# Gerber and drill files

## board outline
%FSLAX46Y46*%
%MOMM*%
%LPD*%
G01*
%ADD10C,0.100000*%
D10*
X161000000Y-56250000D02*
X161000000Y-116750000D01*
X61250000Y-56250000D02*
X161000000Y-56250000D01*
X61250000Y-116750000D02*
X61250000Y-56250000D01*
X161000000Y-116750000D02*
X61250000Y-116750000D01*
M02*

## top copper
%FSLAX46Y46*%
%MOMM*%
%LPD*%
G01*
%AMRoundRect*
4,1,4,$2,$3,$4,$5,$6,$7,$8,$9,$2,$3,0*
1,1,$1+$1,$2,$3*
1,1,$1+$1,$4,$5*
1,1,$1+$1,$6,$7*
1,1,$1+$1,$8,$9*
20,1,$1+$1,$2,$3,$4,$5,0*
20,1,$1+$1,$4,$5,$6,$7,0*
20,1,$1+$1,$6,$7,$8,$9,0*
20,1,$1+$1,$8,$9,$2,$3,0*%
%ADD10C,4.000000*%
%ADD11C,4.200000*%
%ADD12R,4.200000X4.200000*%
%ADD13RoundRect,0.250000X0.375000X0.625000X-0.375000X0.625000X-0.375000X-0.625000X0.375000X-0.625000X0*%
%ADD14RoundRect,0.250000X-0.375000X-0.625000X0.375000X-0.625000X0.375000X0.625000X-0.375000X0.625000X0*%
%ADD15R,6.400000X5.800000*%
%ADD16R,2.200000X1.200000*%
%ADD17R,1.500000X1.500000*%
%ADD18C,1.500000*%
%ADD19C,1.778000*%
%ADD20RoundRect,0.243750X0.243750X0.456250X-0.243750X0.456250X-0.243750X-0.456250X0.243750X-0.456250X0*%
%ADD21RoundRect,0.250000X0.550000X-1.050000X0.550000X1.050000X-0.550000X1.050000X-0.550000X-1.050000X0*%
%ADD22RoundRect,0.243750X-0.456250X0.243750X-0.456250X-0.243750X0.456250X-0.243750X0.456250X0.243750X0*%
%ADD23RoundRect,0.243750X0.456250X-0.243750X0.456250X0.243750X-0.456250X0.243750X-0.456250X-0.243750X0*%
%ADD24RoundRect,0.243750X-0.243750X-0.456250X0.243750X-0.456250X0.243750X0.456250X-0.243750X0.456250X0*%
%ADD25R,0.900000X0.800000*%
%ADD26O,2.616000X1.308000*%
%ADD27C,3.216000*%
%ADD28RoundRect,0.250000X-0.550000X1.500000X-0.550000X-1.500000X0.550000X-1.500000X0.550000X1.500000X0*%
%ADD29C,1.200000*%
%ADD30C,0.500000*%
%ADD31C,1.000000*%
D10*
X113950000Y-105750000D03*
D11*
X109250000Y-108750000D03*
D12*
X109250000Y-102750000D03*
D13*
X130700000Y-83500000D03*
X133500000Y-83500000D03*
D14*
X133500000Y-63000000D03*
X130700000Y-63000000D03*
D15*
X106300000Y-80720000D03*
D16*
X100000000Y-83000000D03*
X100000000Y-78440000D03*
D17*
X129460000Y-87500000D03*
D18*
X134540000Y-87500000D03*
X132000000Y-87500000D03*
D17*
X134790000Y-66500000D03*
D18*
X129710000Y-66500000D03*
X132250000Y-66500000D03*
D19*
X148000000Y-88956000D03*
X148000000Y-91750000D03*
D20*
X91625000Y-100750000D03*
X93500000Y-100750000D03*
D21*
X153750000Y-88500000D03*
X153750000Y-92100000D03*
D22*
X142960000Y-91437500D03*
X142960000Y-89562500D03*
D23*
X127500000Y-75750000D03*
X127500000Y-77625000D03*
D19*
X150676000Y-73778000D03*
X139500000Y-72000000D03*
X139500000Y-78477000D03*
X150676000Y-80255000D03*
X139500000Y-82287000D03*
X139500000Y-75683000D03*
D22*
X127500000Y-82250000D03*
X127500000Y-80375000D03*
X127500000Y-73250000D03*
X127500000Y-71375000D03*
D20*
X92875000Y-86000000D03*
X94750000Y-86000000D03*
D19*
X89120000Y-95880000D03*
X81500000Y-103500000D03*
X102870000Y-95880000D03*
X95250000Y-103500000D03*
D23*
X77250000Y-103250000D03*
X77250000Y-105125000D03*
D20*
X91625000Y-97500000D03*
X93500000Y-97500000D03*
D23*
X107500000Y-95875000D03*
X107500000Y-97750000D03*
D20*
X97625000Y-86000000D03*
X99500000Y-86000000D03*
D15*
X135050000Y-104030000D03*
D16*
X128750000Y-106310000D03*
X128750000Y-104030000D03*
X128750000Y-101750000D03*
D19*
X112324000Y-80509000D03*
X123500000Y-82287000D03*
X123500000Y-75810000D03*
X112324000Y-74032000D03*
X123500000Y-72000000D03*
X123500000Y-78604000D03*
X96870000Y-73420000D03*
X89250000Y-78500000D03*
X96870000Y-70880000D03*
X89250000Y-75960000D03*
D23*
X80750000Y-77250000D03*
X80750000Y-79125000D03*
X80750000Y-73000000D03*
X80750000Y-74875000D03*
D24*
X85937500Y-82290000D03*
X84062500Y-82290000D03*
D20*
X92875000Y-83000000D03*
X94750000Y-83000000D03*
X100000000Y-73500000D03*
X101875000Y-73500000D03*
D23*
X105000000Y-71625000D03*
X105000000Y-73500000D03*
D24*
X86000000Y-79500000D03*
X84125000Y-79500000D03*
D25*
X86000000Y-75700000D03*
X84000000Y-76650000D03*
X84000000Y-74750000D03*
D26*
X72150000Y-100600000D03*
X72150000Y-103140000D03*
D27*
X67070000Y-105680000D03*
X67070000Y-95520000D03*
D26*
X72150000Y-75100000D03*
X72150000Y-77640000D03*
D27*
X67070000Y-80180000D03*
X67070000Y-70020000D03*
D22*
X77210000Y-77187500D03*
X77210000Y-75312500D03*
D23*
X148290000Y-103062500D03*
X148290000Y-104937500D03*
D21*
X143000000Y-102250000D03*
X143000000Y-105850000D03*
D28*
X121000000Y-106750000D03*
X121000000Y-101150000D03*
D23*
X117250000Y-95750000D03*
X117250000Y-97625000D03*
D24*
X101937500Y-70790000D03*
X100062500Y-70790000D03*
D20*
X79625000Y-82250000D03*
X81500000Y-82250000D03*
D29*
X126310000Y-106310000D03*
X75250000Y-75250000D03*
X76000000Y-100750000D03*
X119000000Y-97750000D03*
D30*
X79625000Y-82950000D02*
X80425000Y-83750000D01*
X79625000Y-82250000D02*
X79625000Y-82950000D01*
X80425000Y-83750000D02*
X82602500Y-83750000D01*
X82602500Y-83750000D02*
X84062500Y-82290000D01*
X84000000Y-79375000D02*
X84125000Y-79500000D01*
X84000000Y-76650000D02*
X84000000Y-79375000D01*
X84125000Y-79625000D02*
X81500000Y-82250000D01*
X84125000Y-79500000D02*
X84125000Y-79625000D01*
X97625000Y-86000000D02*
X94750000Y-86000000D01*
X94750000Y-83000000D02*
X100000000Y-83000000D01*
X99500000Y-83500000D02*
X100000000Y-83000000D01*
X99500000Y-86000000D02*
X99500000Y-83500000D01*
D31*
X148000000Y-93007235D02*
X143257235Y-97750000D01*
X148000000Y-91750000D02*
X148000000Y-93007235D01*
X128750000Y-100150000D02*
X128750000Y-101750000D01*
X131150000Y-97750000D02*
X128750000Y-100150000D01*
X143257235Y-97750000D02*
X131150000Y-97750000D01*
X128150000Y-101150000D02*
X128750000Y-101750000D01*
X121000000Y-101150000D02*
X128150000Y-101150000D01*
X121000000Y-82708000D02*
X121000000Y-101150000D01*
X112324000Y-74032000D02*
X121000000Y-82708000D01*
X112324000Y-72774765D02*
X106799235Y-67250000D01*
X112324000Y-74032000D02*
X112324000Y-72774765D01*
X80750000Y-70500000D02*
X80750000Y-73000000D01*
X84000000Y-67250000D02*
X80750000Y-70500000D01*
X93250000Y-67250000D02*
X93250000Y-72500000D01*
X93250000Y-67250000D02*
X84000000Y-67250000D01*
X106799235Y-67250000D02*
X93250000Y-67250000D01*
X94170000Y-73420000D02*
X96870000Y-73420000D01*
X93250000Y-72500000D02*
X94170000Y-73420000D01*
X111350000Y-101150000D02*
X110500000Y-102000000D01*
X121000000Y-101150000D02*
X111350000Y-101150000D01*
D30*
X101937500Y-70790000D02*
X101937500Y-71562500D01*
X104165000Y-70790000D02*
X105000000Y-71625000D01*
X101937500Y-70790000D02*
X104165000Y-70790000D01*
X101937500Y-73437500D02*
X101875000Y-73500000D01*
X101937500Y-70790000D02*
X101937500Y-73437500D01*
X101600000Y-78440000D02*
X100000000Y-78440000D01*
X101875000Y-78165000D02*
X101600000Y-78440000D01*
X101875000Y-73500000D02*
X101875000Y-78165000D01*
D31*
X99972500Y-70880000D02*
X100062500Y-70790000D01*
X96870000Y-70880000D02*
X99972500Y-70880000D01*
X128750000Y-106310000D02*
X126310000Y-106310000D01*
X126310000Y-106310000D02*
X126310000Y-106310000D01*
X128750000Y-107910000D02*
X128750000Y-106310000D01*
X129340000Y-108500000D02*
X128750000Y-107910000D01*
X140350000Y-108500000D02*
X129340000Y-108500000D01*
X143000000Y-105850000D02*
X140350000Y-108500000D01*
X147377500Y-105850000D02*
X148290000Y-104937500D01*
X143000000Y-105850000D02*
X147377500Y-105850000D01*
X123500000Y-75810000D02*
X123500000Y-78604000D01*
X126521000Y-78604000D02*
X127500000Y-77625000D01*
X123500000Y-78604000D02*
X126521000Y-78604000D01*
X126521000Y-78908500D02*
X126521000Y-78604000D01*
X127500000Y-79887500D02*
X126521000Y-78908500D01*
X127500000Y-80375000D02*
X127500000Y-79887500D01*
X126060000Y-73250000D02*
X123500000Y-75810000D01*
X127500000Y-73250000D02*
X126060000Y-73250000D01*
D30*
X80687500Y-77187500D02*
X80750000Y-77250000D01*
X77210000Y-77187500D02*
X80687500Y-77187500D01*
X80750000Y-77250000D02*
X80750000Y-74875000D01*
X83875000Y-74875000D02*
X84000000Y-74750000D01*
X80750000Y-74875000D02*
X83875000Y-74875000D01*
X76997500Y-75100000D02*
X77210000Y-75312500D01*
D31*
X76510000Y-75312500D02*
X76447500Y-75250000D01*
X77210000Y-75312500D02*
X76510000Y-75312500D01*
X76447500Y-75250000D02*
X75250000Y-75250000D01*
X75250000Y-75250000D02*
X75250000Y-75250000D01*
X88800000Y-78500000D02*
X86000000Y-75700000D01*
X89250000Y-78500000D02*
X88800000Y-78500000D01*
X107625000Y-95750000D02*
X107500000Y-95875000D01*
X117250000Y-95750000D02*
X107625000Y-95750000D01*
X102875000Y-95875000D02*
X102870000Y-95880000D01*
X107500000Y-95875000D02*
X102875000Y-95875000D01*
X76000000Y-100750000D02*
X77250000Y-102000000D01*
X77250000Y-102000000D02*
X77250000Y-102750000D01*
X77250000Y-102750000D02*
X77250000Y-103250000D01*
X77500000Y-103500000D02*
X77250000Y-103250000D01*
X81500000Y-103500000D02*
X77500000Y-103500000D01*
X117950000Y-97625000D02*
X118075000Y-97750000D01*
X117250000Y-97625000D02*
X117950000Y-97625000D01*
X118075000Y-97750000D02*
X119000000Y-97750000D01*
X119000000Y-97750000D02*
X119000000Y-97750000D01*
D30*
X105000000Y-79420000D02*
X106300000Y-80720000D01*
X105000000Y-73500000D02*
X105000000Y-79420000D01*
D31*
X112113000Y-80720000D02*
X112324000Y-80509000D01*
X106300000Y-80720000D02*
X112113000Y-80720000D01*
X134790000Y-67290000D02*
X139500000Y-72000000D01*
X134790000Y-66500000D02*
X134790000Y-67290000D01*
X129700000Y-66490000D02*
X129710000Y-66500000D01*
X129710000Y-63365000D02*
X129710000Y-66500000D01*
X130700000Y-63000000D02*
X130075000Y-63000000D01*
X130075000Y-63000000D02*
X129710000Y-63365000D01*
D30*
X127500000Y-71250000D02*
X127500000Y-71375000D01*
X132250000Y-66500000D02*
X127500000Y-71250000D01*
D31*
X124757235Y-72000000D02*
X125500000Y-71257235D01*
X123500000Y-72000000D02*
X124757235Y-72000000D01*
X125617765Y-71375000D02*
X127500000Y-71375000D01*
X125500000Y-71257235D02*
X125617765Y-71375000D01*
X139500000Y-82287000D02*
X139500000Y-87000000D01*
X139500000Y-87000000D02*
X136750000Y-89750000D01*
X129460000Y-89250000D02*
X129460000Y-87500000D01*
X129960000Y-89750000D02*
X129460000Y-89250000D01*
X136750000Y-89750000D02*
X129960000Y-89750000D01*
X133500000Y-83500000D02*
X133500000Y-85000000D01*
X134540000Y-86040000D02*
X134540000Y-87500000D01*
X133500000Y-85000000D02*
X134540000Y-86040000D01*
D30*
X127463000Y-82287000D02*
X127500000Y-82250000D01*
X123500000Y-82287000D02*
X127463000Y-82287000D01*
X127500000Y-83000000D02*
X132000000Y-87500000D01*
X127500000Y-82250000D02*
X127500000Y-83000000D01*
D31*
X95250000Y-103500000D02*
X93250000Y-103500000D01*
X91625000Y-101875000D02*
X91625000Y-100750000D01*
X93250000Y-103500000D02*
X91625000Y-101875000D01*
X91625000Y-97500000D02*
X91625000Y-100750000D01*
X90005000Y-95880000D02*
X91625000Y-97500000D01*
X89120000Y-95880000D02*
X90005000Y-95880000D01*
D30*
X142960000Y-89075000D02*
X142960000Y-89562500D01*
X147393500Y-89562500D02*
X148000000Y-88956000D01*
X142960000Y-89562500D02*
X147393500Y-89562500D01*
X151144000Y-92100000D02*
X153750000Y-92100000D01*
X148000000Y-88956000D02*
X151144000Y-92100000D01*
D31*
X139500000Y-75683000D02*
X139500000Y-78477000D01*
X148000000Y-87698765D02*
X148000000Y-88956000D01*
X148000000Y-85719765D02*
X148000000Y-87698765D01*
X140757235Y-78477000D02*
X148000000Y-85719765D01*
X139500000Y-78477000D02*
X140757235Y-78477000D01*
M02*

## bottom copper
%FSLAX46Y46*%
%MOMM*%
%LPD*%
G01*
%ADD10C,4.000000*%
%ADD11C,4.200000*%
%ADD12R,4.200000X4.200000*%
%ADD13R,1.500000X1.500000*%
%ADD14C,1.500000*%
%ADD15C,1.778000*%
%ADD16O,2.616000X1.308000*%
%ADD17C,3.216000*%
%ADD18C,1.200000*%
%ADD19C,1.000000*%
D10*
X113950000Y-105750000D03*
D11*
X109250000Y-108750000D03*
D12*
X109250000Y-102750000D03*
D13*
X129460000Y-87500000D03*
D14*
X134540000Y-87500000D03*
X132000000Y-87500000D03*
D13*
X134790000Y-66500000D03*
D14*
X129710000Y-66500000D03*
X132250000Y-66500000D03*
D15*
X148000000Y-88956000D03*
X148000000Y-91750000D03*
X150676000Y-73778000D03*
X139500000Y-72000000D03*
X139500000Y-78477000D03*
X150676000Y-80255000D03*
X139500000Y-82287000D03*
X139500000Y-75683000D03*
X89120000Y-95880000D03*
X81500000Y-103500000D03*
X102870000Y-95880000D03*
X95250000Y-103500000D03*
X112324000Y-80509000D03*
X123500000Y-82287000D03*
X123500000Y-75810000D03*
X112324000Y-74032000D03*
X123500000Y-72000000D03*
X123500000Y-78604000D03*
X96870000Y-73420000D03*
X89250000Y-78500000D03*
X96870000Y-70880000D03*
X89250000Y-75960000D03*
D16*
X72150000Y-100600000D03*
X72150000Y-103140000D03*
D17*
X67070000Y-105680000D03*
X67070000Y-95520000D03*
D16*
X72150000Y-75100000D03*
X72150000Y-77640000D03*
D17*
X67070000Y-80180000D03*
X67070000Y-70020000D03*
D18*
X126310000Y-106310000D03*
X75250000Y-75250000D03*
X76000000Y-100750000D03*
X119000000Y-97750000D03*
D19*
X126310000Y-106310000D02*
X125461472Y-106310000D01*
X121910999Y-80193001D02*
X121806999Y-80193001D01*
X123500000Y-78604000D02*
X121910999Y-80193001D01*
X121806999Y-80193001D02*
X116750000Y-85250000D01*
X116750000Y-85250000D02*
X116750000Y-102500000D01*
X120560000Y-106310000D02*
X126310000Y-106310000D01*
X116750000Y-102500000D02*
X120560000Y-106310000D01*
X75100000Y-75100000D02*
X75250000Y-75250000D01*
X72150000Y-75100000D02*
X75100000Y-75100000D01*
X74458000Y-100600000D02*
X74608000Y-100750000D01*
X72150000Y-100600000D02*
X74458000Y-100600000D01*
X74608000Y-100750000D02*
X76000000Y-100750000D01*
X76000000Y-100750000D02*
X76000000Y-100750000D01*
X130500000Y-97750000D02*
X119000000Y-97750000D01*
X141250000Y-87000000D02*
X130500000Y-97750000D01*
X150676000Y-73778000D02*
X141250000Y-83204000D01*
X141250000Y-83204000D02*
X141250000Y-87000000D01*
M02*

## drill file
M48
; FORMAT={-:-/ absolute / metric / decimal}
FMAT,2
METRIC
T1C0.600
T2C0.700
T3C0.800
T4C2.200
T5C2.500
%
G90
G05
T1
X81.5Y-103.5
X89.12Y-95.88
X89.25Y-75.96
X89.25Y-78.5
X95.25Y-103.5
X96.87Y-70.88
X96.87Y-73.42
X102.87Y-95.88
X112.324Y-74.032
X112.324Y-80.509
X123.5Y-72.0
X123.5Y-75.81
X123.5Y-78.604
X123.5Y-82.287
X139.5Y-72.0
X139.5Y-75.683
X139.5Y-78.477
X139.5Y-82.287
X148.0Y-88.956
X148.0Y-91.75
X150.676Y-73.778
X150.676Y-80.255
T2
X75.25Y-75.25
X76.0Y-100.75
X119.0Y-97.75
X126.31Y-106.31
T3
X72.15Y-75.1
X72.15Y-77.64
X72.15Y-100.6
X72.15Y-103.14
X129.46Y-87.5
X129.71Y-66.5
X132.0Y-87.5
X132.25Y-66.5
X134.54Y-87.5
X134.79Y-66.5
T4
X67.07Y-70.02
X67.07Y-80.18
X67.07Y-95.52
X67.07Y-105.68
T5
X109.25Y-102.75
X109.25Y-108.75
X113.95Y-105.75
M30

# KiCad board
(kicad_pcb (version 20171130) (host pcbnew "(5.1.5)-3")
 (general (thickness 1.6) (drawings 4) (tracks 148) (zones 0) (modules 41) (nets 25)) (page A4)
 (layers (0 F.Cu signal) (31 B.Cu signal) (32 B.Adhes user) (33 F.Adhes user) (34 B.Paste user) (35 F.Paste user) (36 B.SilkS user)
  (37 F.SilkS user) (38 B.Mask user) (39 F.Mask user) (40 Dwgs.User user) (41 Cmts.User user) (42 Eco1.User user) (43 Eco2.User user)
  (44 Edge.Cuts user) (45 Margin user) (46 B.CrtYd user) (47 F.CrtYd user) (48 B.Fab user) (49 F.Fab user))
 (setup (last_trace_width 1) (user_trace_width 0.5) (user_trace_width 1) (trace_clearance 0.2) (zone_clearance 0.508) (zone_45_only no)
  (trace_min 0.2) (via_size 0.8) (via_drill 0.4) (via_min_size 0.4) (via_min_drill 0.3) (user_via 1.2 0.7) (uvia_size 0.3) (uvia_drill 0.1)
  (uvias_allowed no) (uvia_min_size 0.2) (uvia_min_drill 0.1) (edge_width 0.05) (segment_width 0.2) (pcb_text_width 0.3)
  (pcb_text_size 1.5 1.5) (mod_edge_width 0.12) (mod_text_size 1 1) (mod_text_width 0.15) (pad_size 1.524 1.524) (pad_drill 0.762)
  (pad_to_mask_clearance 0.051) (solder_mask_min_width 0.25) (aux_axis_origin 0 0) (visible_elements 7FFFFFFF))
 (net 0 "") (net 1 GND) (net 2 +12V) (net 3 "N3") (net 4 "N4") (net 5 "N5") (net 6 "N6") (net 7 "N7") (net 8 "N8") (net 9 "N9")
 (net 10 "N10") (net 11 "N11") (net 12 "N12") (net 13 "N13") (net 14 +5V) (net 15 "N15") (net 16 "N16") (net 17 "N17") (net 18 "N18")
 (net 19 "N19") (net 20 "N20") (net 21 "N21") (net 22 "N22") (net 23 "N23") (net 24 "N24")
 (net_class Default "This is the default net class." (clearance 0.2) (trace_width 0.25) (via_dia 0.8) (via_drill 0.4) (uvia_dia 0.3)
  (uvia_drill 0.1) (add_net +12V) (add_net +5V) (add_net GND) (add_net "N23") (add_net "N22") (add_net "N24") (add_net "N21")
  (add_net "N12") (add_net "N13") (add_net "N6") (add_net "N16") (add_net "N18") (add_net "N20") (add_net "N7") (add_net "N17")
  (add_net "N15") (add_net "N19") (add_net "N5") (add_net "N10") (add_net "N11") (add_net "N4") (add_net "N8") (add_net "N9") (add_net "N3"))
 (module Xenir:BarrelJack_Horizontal (layer F.Cu) (at 109.25 102.75)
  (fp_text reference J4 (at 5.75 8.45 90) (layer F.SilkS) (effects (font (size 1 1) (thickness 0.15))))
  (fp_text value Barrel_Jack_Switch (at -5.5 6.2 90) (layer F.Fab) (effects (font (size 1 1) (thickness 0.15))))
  (pad 3 thru_hole circle (at 4.7 3) (size 4 4) (drill 2.5) (layers *.Cu *.Mask))
  (pad 2 thru_hole circle (at 0 6) (size 4.2 4.2) (drill 2.5) (layers *.Cu *.Mask) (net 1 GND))
  (pad 1 thru_hole rect (at 0 0) (size 4.2 4.2) (drill 2.5) (layers *.Cu *.Mask) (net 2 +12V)))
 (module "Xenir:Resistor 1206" (layer F.Cu) (at 131.973 85.877 180)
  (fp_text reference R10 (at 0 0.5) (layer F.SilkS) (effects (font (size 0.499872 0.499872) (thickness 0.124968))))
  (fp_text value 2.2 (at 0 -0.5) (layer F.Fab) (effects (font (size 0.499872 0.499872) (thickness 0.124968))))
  (pad 2 smd roundrect (at 1.273 2.377 180) (size 1.25 1.75) (layers F.Cu F.Paste F.Mask) (roundrect_rratio 0.2) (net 1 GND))
  (pad 1 smd roundrect (at -1.527 2.377 180) (size 1.25 1.75) (layers F.Cu F.Paste F.Mask) (roundrect_rratio 0.2) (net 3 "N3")))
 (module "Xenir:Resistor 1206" (layer F.Cu) (at 132.227 60.623)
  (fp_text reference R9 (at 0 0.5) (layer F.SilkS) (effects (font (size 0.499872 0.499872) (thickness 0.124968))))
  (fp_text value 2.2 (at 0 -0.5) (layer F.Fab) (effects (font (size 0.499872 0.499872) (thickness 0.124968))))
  (pad 2 smd roundrect (at 1.273 2.377) (size 1.25 1.75) (layers F.Cu F.Paste F.Mask) (roundrect_rratio 0.2) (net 1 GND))
  (pad 1 smd roundrect (at -1.527 2.377) (size 1.25 1.75) (layers F.Cu F.Paste F.Mask) (roundrect_rratio 0.2) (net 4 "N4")))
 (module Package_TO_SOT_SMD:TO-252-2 (layer F.Cu) (at 104.2 80.72)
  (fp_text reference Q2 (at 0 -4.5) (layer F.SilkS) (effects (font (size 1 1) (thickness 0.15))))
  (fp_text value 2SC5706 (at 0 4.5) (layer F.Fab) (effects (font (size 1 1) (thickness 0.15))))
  (pad "" smd rect (at 0.425 1.525) (size 3.05 2.75) (layers F.Paste))
  (pad "" smd rect (at 3.775 -1.525) (size 3.05 2.75) (layers F.Paste))
  (pad "" smd rect (at 0.425 -1.525) (size 3.05 2.75) (layers F.Paste))
  (pad "" smd rect (at 3.775 1.525) (size 3.05 2.75) (layers F.Paste))
  (pad 2 smd rect (at 2.1 0) (size 6.4 5.8) (layers F.Cu F.Mask) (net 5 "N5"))
  (pad 3 smd rect (at -4.2 2.28) (size 2.2 1.2) (layers F.Cu F.Paste F.Mask) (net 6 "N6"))
  (pad 1 smd rect (at -4.2 -2.28) (size 2.2 1.2) (layers F.Cu F.Paste F.Mask) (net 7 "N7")))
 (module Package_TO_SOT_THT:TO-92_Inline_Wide (layer F.Cu) (at 129.46 87.5)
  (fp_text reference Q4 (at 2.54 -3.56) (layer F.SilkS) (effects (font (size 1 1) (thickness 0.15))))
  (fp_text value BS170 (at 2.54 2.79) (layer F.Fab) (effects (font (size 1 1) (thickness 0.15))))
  (pad 1 thru_hole rect (at 0 0 90) (size 1.5 1.5) (drill 0.8) (layers *.Cu *.Mask) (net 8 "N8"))
  (pad 3 thru_hole circle (at 5.08 0 90) (size 1.5 1.5) (drill 0.8) (layers *.Cu *.Mask) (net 3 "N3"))
  (pad 2 thru_hole circle (at 2.54 0 90) (size 1.5 1.5) (drill 0.8) (layers *.Cu *.Mask) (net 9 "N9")))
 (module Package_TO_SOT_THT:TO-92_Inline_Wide (layer F.Cu) (at 134.79 66.5 180)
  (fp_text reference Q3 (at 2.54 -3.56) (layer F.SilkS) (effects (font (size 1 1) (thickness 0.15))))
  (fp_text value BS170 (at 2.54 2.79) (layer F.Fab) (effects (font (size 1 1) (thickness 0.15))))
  (pad 1 thru_hole rect (at 0 0 270) (size 1.5 1.5) (drill 0.8) (layers *.Cu *.Mask) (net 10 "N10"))
  (pad 3 thru_hole circle (at 5.08 0 270) (size 1.5 1.5) (drill 0.8) (layers *.Cu *.Mask) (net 4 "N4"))
  (pad 2 thru_hole circle (at 2.54 0 270) (size 1.5 1.5) (drill 0.8) (layers *.Cu *.Mask) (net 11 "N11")))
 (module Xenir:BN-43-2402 (layer F.Cu) (at 148 95.687 180)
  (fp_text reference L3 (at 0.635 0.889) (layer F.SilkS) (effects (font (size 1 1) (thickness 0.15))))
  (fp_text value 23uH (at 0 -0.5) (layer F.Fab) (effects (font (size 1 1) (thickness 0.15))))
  (pad 2 thru_hole circle (at 0 6.731 180) (size 1.778 1.778) (drill 0.6) (layers *.Cu *.Mask) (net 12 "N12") (solder_mask_margin 0.1016))
  (pad 1 thru_hole circle (at 0 3.937 180) (size 1.778 1.778) (drill 0.6) (layers *.Cu *.Mask) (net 2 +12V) (solder_mask_margin 0.1016)))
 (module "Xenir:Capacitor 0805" (layer F.Cu) (at 92.5625 103.29 180)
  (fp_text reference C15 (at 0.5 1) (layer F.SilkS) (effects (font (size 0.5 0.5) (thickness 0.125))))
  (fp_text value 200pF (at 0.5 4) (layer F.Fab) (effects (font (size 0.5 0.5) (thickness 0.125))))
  (pad 2 smd roundrect (at 0.9375 2.54 180) (size 0.975 1.4) (layers F.Cu F.Paste F.Mask) (roundrect_rratio 0.25) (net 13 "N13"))
  (pad 1 smd roundrect (at -0.9375 2.54 180) (size 0.975 1.4) (layers F.Cu F.Paste F.Mask) (roundrect_rratio 0.25) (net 1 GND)))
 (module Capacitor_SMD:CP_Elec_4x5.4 (layer F.Cu) (at 153.75 90.3 90)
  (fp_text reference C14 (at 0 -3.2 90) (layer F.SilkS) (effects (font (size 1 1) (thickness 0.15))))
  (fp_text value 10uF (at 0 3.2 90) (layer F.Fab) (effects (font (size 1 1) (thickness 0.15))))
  (pad 2 smd roundrect (at 1.8 0 90) (size 2.6 1.6) (layers F.Cu F.Paste F.Mask) (roundrect_rratio 0.15625) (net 1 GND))
  (pad 1 smd roundrect (at -1.8 0 90) (size 2.6 1.6) (layers F.Cu F.Paste F.Mask) (roundrect_rratio 0.15625) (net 12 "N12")))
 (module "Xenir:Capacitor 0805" (layer F.Cu) (at 145.5 90.5 270)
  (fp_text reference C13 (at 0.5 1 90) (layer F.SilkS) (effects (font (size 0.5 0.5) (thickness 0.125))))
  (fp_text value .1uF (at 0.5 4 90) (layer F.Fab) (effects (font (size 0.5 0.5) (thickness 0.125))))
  (pad 2 smd roundrect (at 0.9375 2.54 270) (size 0.975 1.4) (layers F.Cu F.Paste F.Mask) (roundrect_rratio 0.25) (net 1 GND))
  (pad 1 smd roundrect (at -0.9375 2.54 270) (size 0.975 1.4) (layers F.Cu F.Paste F.Mask) (roundrect_rratio 0.25) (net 12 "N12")))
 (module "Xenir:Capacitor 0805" (layer F.Cu) (at 124.96 76.6875 90)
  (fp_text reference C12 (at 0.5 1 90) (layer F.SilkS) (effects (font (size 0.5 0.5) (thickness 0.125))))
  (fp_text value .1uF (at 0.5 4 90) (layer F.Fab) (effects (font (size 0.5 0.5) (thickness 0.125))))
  (pad 2 smd roundrect (at 0.9375 2.54 90) (size 0.975 1.4) (layers F.Cu F.Paste F.Mask) (roundrect_rratio 0.25) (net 1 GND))
  (pad 1 smd roundrect (at -0.9375 2.54 90) (size 0.975 1.4) (layers F.Cu F.Paste F.Mask) (roundrect_rratio 0.25) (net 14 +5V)))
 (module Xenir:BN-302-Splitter (layer F.Cu) (at 145.088 85.843 180)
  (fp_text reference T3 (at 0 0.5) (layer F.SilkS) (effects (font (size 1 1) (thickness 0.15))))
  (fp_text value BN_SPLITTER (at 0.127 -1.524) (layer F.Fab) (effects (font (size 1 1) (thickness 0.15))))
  (pad C1B thru_hole circle (at -5.588 12.065 180) (size 1.778 1.778) (drill 0.6) (layers *.Cu *.Mask) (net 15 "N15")
   (solder_mask_margin 0.1016))
  (pad C3B thru_hole circle (at 5.588 13.843 180) (size 1.778 1.778) (drill 0.6) (layers *.Cu *.Mask) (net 10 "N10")
   (solder_mask_margin 0.1016))
  (pad C2B thru_hole circle (at 5.588 7.366 180) (size 1.778 1.778) (drill 0.6) (layers *.Cu *.Mask) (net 12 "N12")
   (solder_mask_margin 0.1016))
  (pad C1A thru_hole circle (at -5.588 5.588 180) (size 1.778 1.778) (drill 0.6) (layers *.Cu *.Mask) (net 1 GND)
   (solder_mask_margin 0.1016))
  (pad C2A thru_hole circle (at 5.588 3.556 180) (size 1.778 1.778) (drill 0.6) (layers *.Cu *.Mask) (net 8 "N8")
   (solder_mask_margin 0.1016))
  (pad C3A thru_hole circle (at 5.588 10.16 180) (size 1.778 1.778) (drill 0.6) (layers *.Cu *.Mask) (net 12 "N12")
   (solder_mask_margin 0.1016)))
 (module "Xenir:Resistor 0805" (layer F.Cu) (at 130.04 81.3125 270)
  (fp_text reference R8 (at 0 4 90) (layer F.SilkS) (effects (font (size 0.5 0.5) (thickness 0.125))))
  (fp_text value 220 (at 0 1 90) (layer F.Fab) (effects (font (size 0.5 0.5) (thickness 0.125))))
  (pad 2 smd roundrect (at 0.9375 2.54 270) (size 0.975 1.4) (layers F.Cu F.Paste F.Mask) (roundrect_rratio 0.25) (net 9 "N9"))
  (pad 1 smd roundrect (at -0.9375 2.54 270) (size 0.975 1.4) (layers F.Cu F.Paste F.Mask) (roundrect_rratio 0.25) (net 14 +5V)))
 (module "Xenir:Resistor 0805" (layer F.Cu) (at 130.04 72.3125 270)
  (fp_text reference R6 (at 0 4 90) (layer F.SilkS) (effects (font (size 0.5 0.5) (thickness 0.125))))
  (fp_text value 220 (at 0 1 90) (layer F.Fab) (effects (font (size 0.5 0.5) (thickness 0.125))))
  (pad 2 smd roundrect (at 0.9375 2.54 270) (size 0.975 1.4) (layers F.Cu F.Paste F.Mask) (roundrect_rratio 0.25) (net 14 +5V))
  (pad 1 smd roundrect (at -0.9375 2.54 270) (size 0.975 1.4) (layers F.Cu F.Paste F.Mask) (roundrect_rratio 0.25) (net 11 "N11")))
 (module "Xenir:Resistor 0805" (layer F.Cu) (at 93.8125 88.54 180)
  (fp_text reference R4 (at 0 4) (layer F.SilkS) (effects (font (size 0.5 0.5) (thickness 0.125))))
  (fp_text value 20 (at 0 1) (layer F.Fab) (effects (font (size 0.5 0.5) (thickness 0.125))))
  (pad 2 smd roundrect (at 0.9375 2.54 180) (size 0.975 1.4) (layers F.Cu F.Paste F.Mask) (roundrect_rratio 0.25) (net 1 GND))
  (pad 1 smd roundrect (at -0.9375 2.54 180) (size 0.975 1.4) (layers F.Cu F.Paste F.Mask) (roundrect_rratio 0.25) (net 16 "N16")))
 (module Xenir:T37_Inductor (layer F.Cu) (at 85.31 106.69 180)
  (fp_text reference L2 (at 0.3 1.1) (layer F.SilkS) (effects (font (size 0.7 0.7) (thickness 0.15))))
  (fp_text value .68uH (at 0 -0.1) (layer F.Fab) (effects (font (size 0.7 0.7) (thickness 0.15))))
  (pad 1 thru_hole circle (at -3.81 10.81 180) (size 1.778 1.778) (drill 0.6) (layers *.Cu *.Mask) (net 13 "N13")
   (solder_mask_margin 0.1016))
  (pad 2 thru_hole circle (at 3.81 3.19 180) (size 1.778 1.778) (drill 0.6) (layers *.Cu *.Mask) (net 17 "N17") (solder_mask_margin 0.1016)))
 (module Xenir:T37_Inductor (layer F.Cu) (at 99.06 106.69 180)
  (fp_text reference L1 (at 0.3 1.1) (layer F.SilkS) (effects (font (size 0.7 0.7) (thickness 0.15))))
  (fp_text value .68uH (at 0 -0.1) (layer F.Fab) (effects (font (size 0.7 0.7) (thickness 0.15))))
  (pad 1 thru_hole circle (at -3.81 10.81 180) (size 1.778 1.778) (drill 0.6) (layers *.Cu *.Mask) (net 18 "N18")
   (solder_mask_margin 0.1016))
  (pad 2 thru_hole circle (at 3.81 3.19 180) (size 1.778 1.778) (drill 0.6) (layers *.Cu *.Mask) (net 13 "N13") (solder_mask_margin 0.1016)))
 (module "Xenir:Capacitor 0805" (layer F.Cu) (at 74.71 104.1875 90)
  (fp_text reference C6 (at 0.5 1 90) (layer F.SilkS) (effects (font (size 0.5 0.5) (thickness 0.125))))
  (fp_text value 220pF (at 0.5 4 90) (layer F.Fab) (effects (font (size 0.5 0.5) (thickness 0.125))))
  (pad 2 smd roundrect (at 0.9375 2.54 90) (size 0.975 1.4) (layers F.Cu F.Paste F.Mask) (roundrect_rratio 0.25) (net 17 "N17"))
  (pad 1 smd roundrect (at -0.9375 2.54 90) (size 0.975 1.4) (layers F.Cu F.Paste F.Mask) (roundrect_rratio 0.25) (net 1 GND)))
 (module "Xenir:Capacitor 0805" (layer F.Cu) (at 92.5625 100.04 180)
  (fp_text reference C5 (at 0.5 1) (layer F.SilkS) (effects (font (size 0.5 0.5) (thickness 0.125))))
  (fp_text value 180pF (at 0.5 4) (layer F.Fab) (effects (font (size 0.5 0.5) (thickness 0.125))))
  (pad 2 smd roundrect (at 0.9375 2.54 180) (size 0.975 1.4) (layers F.Cu F.Paste F.Mask) (roundrect_rratio 0.25) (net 13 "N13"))
  (pad 1 smd roundrect (at -0.9375 2.54 180) (size 0.975 1.4) (layers F.Cu F.Paste F.Mask) (roundrect_rratio 0.25) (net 1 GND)))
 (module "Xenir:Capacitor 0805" (layer F.Cu) (at 104.96 96.8125 90)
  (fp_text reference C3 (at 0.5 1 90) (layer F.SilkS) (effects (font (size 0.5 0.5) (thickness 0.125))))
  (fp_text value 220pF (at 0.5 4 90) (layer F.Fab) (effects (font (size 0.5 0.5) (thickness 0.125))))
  (pad 2 smd roundrect (at 0.9375 2.54 90) (size 0.975 1.4) (layers F.Cu F.Paste F.Mask) (roundrect_rratio 0.25) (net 18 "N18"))
  (pad 1 smd roundrect (at -0.9375 2.54 90) (size 0.975 1.4) (layers F.Cu F.Paste F.Mask) (roundrect_rratio 0.25) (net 1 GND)))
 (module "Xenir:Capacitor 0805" (layer F.Cu) (at 98.5625 88.54 180)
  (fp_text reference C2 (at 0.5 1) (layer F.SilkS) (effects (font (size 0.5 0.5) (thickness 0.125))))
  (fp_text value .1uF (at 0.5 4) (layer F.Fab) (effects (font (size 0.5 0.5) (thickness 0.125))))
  (pad 2 smd roundrect (at 0.9375 2.54 180) (size 0.975 1.4) (layers F.Cu F.Paste F.Mask) (roundrect_rratio 0.25) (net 16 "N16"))
  (pad 1 smd roundrect (at -0.9375 2.54 180) (size 0.975 1.4) (layers F.Cu F.Paste F.Mask) (roundrect_rratio 0.25) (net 6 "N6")))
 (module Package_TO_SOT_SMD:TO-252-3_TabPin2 (layer F.Cu) (at 132.95 104.03)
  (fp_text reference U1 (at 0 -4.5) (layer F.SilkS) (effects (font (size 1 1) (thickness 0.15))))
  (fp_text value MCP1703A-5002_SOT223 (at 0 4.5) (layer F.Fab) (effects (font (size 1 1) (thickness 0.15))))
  (pad "" smd rect (at 0.425 1.525) (size 3.05 2.75) (layers F.Paste))
  (pad "" smd rect (at 3.775 -1.525) (size 3.05 2.75) (layers F.Paste))
  (pad "" smd rect (at 0.425 -1.525) (size 3.05 2.75) (layers F.Paste))
  (pad "" smd rect (at 3.775 1.525) (size 3.05 2.75) (layers F.Paste))
  (pad 2 smd rect (at 2.1 0) (size 6.4 5.8) (layers F.Cu F.Mask) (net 1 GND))
  (pad 3 smd rect (at -4.2 2.28) (size 2.2 1.2) (layers F.Cu F.Paste F.Mask) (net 14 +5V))
  (pad 2 smd rect (at -4.2 0) (size 2.2 1.2) (layers F.Cu F.Paste F.Mask) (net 1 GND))
  (pad 1 smd rect (at -4.2 -2.28) (size 2.2 1.2) (layers F.Cu F.Paste F.Mask) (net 2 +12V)))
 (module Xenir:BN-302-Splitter (layer F.Cu) (at 117.912 68.444)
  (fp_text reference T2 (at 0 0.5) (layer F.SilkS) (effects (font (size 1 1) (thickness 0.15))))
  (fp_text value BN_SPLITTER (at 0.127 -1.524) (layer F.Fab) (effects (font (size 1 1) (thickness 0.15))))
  (pad C1B thru_hole circle (at -5.588 12.065) (size 1.778 1.778) (drill 0.6) (layers *.Cu *.Mask) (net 5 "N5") (solder_mask_margin 0.1016))
  (pad C3B thru_hole circle (at 5.588 13.843) (size 1.778 1.778) (drill 0.6) (layers *.Cu *.Mask) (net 9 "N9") (solder_mask_margin 0.1016))
  (pad C2B thru_hole circle (at 5.588 7.366) (size 1.778 1.778) (drill 0.6) (layers *.Cu *.Mask) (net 14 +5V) (solder_mask_margin 0.1016))
  (pad C1A thru_hole circle (at -5.588 5.588) (size 1.778 1.778) (drill 0.6) (layers *.Cu *.Mask) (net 2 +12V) (solder_mask_margin 0.1016))
  (pad C2A thru_hole circle (at 5.588 3.556) (size 1.778 1.778) (drill 0.6) (layers *.Cu *.Mask) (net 11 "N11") (solder_mask_margin 0.1016))
  (pad C3A thru_hole circle (at 5.588 10.16) (size 1.778 1.778) (drill 0.6) (layers *.Cu *.Mask) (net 14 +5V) (solder_mask_margin 0.1016)))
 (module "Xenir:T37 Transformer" (layer F.Cu) (at 93.06 67.69)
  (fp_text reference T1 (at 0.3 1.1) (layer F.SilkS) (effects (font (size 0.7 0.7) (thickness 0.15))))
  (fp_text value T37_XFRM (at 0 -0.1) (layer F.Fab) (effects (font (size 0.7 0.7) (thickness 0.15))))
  (pad C1B thru_hole circle (at 3.81 5.73) (size 1.778 1.778) (drill 0.6) (layers *.Cu *.Mask) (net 2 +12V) (solder_mask_margin 0.1016))
  (pad C1A thru_hole circle (at -3.81 10.81) (size 1.778 1.778) (drill 0.6) (layers *.Cu *.Mask) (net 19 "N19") (solder_mask_margin 0.1016))
  (pad C2B thru_hole circle (at 3.81 3.19) (size 1.778 1.778) (drill 0.6) (layers *.Cu *.Mask) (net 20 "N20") (solder_mask_margin 0.1016))
  (pad C2A thru_hole circle (at -3.81 8.27) (size 1.778 1.778) (drill 0.6) (layers *.Cu *.Mask) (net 1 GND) (solder_mask_margin 0.1016)))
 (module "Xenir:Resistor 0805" (layer F.Cu) (at 78.21 78.1875 90)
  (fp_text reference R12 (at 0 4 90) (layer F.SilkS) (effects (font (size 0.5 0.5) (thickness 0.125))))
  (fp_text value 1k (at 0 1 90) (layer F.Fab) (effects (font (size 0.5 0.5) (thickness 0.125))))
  (pad 2 smd roundrect (at 0.9375 2.54 90) (size 0.975 1.4) (layers F.Cu F.Paste F.Mask) (roundrect_rratio 0.25) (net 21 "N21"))
  (pad 1 smd roundrect (at -0.9375 2.54 90) (size 0.975 1.4) (layers F.Cu F.Paste F.Mask) (roundrect_rratio 0.25) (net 1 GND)))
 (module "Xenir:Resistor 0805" (layer F.Cu) (at 78.21 73.9375 90)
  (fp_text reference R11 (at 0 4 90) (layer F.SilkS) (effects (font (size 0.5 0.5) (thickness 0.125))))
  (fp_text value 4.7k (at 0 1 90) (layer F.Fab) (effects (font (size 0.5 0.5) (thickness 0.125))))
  (pad 2 smd roundrect (at 0.9375 2.54 90) (size 0.975 1.4) (layers F.Cu F.Paste F.Mask) (roundrect_rratio 0.25) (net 2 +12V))
  (pad 1 smd roundrect (at -0.9375 2.54 90) (size 0.975 1.4) (layers F.Cu F.Paste F.Mask) (roundrect_rratio 0.25) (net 21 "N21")))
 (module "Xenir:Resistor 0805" (layer F.Cu) (at 85 79.75)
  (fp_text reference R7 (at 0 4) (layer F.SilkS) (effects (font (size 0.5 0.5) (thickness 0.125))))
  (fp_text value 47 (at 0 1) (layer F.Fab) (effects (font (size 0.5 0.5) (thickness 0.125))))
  (pad 2 smd roundrect (at 0.9375 2.54) (size 0.975 1.4) (layers F.Cu F.Paste F.Mask) (roundrect_rratio 0.25) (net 1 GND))
  (pad 1 smd roundrect (at -0.9375 2.54) (size 0.975 1.4) (layers F.Cu F.Paste F.Mask) (roundrect_rratio 0.25) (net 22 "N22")))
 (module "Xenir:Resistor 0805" (layer F.Cu) (at 93.8125 85.54 180)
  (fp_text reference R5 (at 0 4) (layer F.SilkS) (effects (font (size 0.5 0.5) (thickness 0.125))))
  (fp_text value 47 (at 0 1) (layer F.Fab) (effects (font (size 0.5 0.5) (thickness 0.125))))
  (pad 2 smd roundrect (at 0.9375 2.54 180) (size 0.975 1.4) (layers F.Cu F.Paste F.Mask) (roundrect_rratio 0.25) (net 1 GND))
  (pad 1 smd roundrect (at -0.9375 2.54 180) (size 0.975 1.4) (layers F.Cu F.Paste F.Mask) (roundrect_rratio 0.25) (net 6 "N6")))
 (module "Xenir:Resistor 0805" (layer F.Cu) (at 100.9375 76.04 180)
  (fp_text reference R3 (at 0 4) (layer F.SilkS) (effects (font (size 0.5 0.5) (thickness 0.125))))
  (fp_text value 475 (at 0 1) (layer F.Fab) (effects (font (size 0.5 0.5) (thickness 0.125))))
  (pad 2 smd roundrect (at 0.9375 2.54 180) (size 0.975 1.4) (layers F.Cu F.Paste F.Mask) (roundrect_rratio 0.25) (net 1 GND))
  (pad 1 smd roundrect (at -0.9375 2.54 180) (size 0.975 1.4) (layers F.Cu F.Paste F.Mask) (roundrect_rratio 0.25) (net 7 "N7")))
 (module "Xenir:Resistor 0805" (layer F.Cu) (at 102.46 72.5625 90)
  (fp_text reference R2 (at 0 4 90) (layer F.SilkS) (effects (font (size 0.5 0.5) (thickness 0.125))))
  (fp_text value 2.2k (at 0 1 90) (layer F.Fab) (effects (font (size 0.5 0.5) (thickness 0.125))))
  (pad 2 smd roundrect (at 0.9375 2.54 90) (size 0.975 1.4) (layers F.Cu F.Paste F.Mask) (roundrect_rratio 0.25) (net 7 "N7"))
  (pad 1 smd roundrect (at -0.9375 2.54 90) (size 0.975 1.4) (layers F.Cu F.Paste F.Mask) (roundrect_rratio 0.25) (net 5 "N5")))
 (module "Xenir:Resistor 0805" (layer F.Cu) (at 85.0625 76.96)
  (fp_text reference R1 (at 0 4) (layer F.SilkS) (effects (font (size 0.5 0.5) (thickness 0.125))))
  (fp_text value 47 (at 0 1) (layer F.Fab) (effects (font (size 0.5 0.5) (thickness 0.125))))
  (pad 2 smd roundrect (at 0.9375 2.54) (size 0.975 1.4) (layers F.Cu F.Paste F.Mask) (roundrect_rratio 0.25) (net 1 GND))
  (pad 1 smd roundrect (at -0.9375 2.54) (size 0.975 1.4) (layers F.Cu F.Paste F.Mask) (roundrect_rratio 0.25) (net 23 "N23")))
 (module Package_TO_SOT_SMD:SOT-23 (layer F.Cu) (at 85 75.7)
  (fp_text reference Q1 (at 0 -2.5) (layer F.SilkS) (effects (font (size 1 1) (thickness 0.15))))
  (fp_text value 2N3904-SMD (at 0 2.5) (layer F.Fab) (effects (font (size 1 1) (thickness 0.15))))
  (pad 3 smd rect (at 1 0) (size 0.9 0.8) (layers F.Cu F.Paste F.Mask) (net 19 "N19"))
  (pad 2 smd rect (at -1 0.95) (size 0.9 0.8) (layers F.Cu F.Paste F.Mask) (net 23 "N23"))
  (pad 1 smd rect (at -1 -0.95) (size 0.9 0.8) (layers F.Cu F.Paste F.Mask) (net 21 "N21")))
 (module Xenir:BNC (layer F.Cu) (at 68.25 100.5 90)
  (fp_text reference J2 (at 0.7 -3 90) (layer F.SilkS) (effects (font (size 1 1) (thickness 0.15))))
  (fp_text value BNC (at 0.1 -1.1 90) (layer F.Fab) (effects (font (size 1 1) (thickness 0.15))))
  (pad S thru_hole oval (at -0.1 3.9 180) (size 2.616 1.308) (drill 0.8) (layers *.Cu *.Mask) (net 17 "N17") (solder_mask_margin 0.1016))
  (pad GND thru_hole oval (at -2.64 3.9 180) (size 2.616 1.308) (drill 0.8) (layers *.Cu *.Mask) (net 1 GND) (solder_mask_margin 0.1016))
  (pad 3 thru_hole circle (at -5.18 -1.18 90) (size 3.216 3.216) (drill 2.2) (layers *.Cu *.Mask) (solder_mask_margin 0.1016))
  (pad 4 thru_hole circle (at 4.98 -1.18 90) (size 3.216 3.216) (drill 2.2) (layers *.Cu *.Mask) (solder_mask_margin 0.1016)))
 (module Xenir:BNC (layer F.Cu) (at 68.25 75 90)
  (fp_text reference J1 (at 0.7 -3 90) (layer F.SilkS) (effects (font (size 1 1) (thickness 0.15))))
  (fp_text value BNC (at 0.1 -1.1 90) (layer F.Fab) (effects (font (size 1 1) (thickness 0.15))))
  (pad S thru_hole oval (at -0.1 3.9 180) (size 2.616 1.308) (drill 0.8) (layers *.Cu *.Mask) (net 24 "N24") (solder_mask_margin 0.1016))
  (pad GND thru_hole oval (at -2.64 3.9 180) (size 2.616 1.308) (drill 0.8) (layers *.Cu *.Mask) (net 1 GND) (solder_mask_margin 0.1016))
  (pad 3 thru_hole circle (at -5.18 -1.18 90) (size 3.216 3.216) (drill 2.2) (layers *.Cu *.Mask) (solder_mask_margin 0.1016))
  (pad 4 thru_hole circle (at 4.98 -1.18 90) (size 3.216 3.216) (drill 2.2) (layers *.Cu *.Mask) (solder_mask_margin 0.1016)))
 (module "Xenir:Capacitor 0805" (layer F.Cu) (at 79.75 76.25 270)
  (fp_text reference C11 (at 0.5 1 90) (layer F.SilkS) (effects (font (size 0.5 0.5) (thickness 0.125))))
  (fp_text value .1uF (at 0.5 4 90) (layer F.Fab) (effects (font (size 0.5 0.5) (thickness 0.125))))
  (pad 2 smd roundrect (at 0.9375 2.54 270) (size 0.975 1.4) (layers F.Cu F.Paste F.Mask) (roundrect_rratio 0.25) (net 21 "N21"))
  (pad 1 smd roundrect (at -0.9375 2.54 270) (size 0.975 1.4) (layers F.Cu F.Paste F.Mask) (roundrect_rratio 0.25) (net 24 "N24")))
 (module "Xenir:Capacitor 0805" (layer F.Cu) (at 145.75 104 90)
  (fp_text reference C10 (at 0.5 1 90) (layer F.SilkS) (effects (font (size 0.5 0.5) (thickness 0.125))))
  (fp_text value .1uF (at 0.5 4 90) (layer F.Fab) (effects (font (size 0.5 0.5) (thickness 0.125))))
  (pad 2 smd roundrect (at 0.9375 2.54 90) (size 0.975 1.4) (layers F.Cu F.Paste F.Mask) (roundrect_rratio 0.25) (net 1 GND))
  (pad 1 smd roundrect (at -0.9375 2.54 90) (size 0.975 1.4) (layers F.Cu F.Paste F.Mask) (roundrect_rratio 0.25) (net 14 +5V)))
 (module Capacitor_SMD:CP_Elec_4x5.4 (layer F.Cu) (at 143 104.05 90)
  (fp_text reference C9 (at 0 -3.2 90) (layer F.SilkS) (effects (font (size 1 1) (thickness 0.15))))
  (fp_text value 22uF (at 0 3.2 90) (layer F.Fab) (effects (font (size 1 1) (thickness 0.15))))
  (pad 2 smd roundrect (at 1.8 0 90) (size 2.6 1.6) (layers F.Cu F.Paste F.Mask) (roundrect_rratio 0.15625) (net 1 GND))
  (pad 1 smd roundrect (at -1.8 0 90) (size 2.6 1.6) (layers F.Cu F.Paste F.Mask) (roundrect_rratio 0.15625) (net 14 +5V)))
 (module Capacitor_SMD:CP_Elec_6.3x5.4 (layer F.Cu) (at 121 103.95 270)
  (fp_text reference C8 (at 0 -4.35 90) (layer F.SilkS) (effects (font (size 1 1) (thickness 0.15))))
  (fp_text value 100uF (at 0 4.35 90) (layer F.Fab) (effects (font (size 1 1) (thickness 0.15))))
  (pad 2 smd roundrect (at 2.8 0 270) (size 3.5 1.6) (layers F.Cu F.Paste F.Mask) (roundrect_rratio 0.15625) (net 1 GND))
  (pad 1 smd roundrect (at -2.8 0 270) (size 3.5 1.6) (layers F.Cu F.Paste F.Mask) (roundrect_rratio 0.15625) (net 2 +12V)))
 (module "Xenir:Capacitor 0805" (layer F.Cu) (at 114.71 96.6875 90)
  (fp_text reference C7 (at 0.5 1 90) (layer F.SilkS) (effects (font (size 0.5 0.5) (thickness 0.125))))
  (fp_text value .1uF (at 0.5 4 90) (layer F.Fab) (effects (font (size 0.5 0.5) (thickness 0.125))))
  (pad 2 smd roundrect (at 0.9375 2.54 90) (size 0.975 1.4) (layers F.Cu F.Paste F.Mask) (roundrect_rratio 0.25) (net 18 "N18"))
  (pad 1 smd roundrect (at -0.9375 2.54 90) (size 0.975 1.4) (layers F.Cu F.Paste F.Mask) (roundrect_rratio 0.25) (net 15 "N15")))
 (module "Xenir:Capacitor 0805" (layer F.Cu) (at 101 68.25)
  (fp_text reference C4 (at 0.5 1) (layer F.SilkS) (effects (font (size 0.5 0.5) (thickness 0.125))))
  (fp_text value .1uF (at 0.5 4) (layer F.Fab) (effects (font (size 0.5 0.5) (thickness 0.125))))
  (pad 2 smd roundrect (at 0.9375 2.54) (size 0.975 1.4) (layers F.Cu F.Paste F.Mask) (roundrect_rratio 0.25) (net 7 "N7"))
  (pad 1 smd roundrect (at -0.9375 2.54) (size 0.975 1.4) (layers F.Cu F.Paste F.Mask) (roundrect_rratio 0.25) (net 20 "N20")))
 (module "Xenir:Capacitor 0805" (layer F.Cu) (at 80.5625 84.79 180)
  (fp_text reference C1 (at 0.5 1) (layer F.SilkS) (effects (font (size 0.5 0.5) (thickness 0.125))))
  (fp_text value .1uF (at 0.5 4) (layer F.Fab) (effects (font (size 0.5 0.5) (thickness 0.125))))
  (pad 2 smd roundrect (at 0.9375 2.54 180) (size 0.975 1.4) (layers F.Cu F.Paste F.Mask) (roundrect_rratio 0.25) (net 22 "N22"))
  (pad 1 smd roundrect (at -0.9375 2.54 180) (size 0.975 1.4) (layers F.Cu F.Paste F.Mask) (roundrect_rratio 0.25) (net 23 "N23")))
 (gr_line (start 161 56.25) (end 161 116.75) (layer Edge.Cuts) (width 0.1))
 (gr_line (start 61.25 56.25) (end 161 56.25) (layer Edge.Cuts) (width 0.1))
 (gr_line (start 61.25 116.75) (end 61.25 56.25) (layer Edge.Cuts) (width 0.1))
 (gr_line (start 161 116.75) (end 61.25 116.75) (layer Edge.Cuts) (width 0.1))
 (segment (start 79.625 82.95) (end 80.425 83.75) (width 0.5) (layer F.Cu) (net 22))
 (segment (start 79.625 82.25) (end 79.625 82.95) (width 0.5) (layer F.Cu) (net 22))
 (segment (start 80.425 83.75) (end 82.6025 83.75) (width 0.5) (layer F.Cu) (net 22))
 (segment (start 82.6025 83.75) (end 84.0625 82.29) (width 0.5) (layer F.Cu) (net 22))
 (segment (start 84 79.375) (end 84.125 79.5) (width 0.5) (layer F.Cu) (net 23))
 (segment (start 84 76.65) (end 84 79.375) (width 0.5) (layer F.Cu) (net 23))
 (segment (start 84.125 79.625) (end 81.5 82.25) (width 0.5) (layer F.Cu) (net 23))
 (segment (start 84.125 79.5) (end 84.125 79.625) (width 0.5) (layer F.Cu) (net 23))
 (segment (start 97.625 86) (end 94.75 86) (width 0.5) (layer F.Cu) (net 16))
 (segment (start 94.75 83) (end 100 83) (width 0.5) (layer F.Cu) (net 6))
 (segment (start 99.5 83.5) (end 100 83) (width 0.5) (layer F.Cu) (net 6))
 (segment (start 99.5 86) (end 99.5 83.5) (width 0.5) (layer F.Cu) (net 6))
 (segment (start 148 93.007235) (end 143.257235 97.75) (width 1) (layer F.Cu) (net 2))
 (segment (start 148 91.75) (end 148 93.007235) (width 1) (layer F.Cu) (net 2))
 (segment (start 128.75 100.15) (end 128.75 101.75) (width 1) (layer F.Cu) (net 2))
 (segment (start 131.15 97.75) (end 128.75 100.15) (width 1) (layer F.Cu) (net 2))
 (segment (start 143.257235 97.75) (end 131.15 97.75) (width 1) (layer F.Cu) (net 2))
 (segment (start 128.15 101.15) (end 128.75 101.75) (width 1) (layer F.Cu) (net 2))
 (segment (start 121 101.15) (end 128.15 101.15) (width 1) (layer F.Cu) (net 2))
 (segment (start 121 82.708) (end 121 101.15) (width 1) (layer F.Cu) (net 2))
 (segment (start 112.324 74.032) (end 121 82.708) (width 1) (layer F.Cu) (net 2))
 (segment (start 112.324 72.774765) (end 106.799235 67.25) (width 1) (layer F.Cu) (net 2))
 (segment (start 112.324 74.032) (end 112.324 72.774765) (width 1) (layer F.Cu) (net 2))
 (segment (start 80.75 70.5) (end 80.75 73) (width 1) (layer F.Cu) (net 2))
 (segment (start 84 67.25) (end 80.75 70.5) (width 1) (layer F.Cu) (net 2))
 (segment (start 93.25 67.25) (end 93.25 72.5) (width 1) (layer F.Cu) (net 2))
 (segment (start 93.25 67.25) (end 84 67.25) (width 1) (layer F.Cu) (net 2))
 (segment (start 106.799235 67.25) (end 93.25 67.25) (width 1) (layer F.Cu) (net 2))
 (segment (start 94.17 73.42) (end 96.87 73.42) (width 1) (layer F.Cu) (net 2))
 (segment (start 93.25 72.5) (end 94.17 73.42) (width 1) (layer F.Cu) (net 2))
 (segment (start 111.35 101.15) (end 110.5 102) (width 1) (layer F.Cu) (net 2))
 (segment (start 121 101.15) (end 111.35 101.15) (width 1) (layer F.Cu) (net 2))
 (segment (start 101.9375 70.79) (end 101.9375 71.5625) (width 0.5) (layer F.Cu) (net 7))
 (segment (start 104.165 70.79) (end 105 71.625) (width 0.5) (layer F.Cu) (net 7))
 (segment (start 101.9375 70.79) (end 104.165 70.79) (width 0.5) (layer F.Cu) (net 7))
 (segment (start 101.9375 73.4375) (end 101.875 73.5) (width 0.5) (layer F.Cu) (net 7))
 (segment (start 101.9375 70.79) (end 101.9375 73.4375) (width 0.5) (layer F.Cu) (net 7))
 (segment (start 101.6 78.44) (end 100 78.44) (width 0.5) (layer F.Cu) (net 7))
 (segment (start 101.875 78.165) (end 101.6 78.44) (width 0.5) (layer F.Cu) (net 7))
 (segment (start 101.875 73.5) (end 101.875 78.165) (width 0.5) (layer F.Cu) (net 7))
 (segment (start 99.9725 70.88) (end 100.0625 70.79) (width 1) (layer F.Cu) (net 20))
 (segment (start 96.87 70.88) (end 99.9725 70.88) (width 1) (layer F.Cu) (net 20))
 (segment (start 128.75 106.31) (end 126.31 106.31) (width 1) (layer F.Cu) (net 14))
 (segment (start 126.31 106.31) (end 126.31 106.31) (width 1) (layer F.Cu) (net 14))
 (via (at 126.31 106.31) (size 1.2) (drill 0.7) (layers F.Cu B.Cu) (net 14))
 (segment (start 126.31 106.31) (end 125.461472 106.31) (width 1) (layer B.Cu) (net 14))
 (segment (start 128.75 107.91) (end 128.75 106.31) (width 1) (layer F.Cu) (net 14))
 (segment (start 129.34 108.5) (end 128.75 107.91) (width 1) (layer F.Cu) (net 14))
 (segment (start 140.35 108.5) (end 129.34 108.5) (width 1) (layer F.Cu) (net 14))
 (segment (start 143 105.85) (end 140.35 108.5) (width 1) (layer F.Cu) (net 14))
 (segment (start 147.3775 105.85) (end 148.29 104.9375) (width 1) (layer F.Cu) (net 14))
 (segment (start 143 105.85) (end 147.3775 105.85) (width 1) (layer F.Cu) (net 14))
 (segment (start 123.5 75.81) (end 123.5 78.604) (width 1) (layer F.Cu) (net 14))
 (segment (start 126.521 78.604) (end 127.5 77.625) (width 1) (layer F.Cu) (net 14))
 (segment (start 123.5 78.604) (end 126.521 78.604) (width 1) (layer F.Cu) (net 14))
 (segment (start 126.521 78.9085) (end 126.521 78.604) (width 1) (layer F.Cu) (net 14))
 (segment (start 127.5 79.8875) (end 126.521 78.9085) (width 1) (layer F.Cu) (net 14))
 (segment (start 127.5 80.375) (end 127.5 79.8875) (width 1) (layer F.Cu) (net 14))
 (segment (start 126.06 73.25) (end 123.5 75.81) (width 1) (layer F.Cu) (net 14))
 (segment (start 127.5 73.25) (end 126.06 73.25) (width 1) (layer F.Cu) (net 14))
 (segment (start 121.910999 80.193001) (end 121.806999 80.193001) (width 1) (layer B.Cu) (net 14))
 (segment (start 123.5 78.604) (end 121.910999 80.193001) (width 1) (layer B.Cu) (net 14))
 (segment (start 121.806999 80.193001) (end 116.75 85.25) (width 1) (layer B.Cu) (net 14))
 (segment (start 116.75 85.25) (end 116.75 102.5) (width 1) (layer B.Cu) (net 14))
 (segment (start 120.56 106.31) (end 126.31 106.31) (width 1) (layer B.Cu) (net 14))
 (segment (start 116.75 102.5) (end 120.56 106.31) (width 1) (layer B.Cu) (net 14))
 (segment (start 80.6875 77.1875) (end 80.75 77.25) (width 0.5) (layer F.Cu) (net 21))
 (segment (start 77.21 77.1875) (end 80.6875 77.1875) (width 0.5) (layer F.Cu) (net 21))
 (segment (start 80.75 77.25) (end 80.75 74.875) (width 0.5) (layer F.Cu) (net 21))
 (segment (start 83.875 74.875) (end 84 74.75) (width 0.5) (layer F.Cu) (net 21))
 (segment (start 80.75 74.875) (end 83.875 74.875) (width 0.5) (layer F.Cu) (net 21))
 (segment (start 76.9975 75.1) (end 77.21 75.3125) (width 0.5) (layer F.Cu) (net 24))
 (segment (start 76.51 75.3125) (end 76.4475 75.25) (width 1) (layer F.Cu) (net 24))
 (segment (start 77.21 75.3125) (end 76.51 75.3125) (width 1) (layer F.Cu) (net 24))
 (segment (start 76.4475 75.25) (end 75.25 75.25) (width 1) (layer F.Cu) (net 24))
 (segment (start 75.25 75.25) (end 75.25 75.25) (width 1) (layer F.Cu) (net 24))
 (via (at 75.25 75.25) (size 1.2) (drill 0.7) (layers F.Cu B.Cu) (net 24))
 (segment (start 75.1 75.1) (end 75.25 75.25) (width 1) (layer B.Cu) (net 24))
 (segment (start 72.15 75.1) (end 75.1 75.1) (width 1) (layer B.Cu) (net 24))
 (segment (start 88.8 78.5) (end 86 75.7) (width 1) (layer F.Cu) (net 19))
 (segment (start 89.25 78.5) (end 88.8 78.5) (width 1) (layer F.Cu) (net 19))
 (segment (start 107.625 95.75) (end 107.5 95.875) (width 1) (layer F.Cu) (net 18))
 (segment (start 117.25 95.75) (end 107.625 95.75) (width 1) (layer F.Cu) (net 18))
 (segment (start 102.875 95.875) (end 102.87 95.88) (width 1) (layer F.Cu) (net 18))
 (segment (start 107.5 95.875) (end 102.875 95.875) (width 1) (layer F.Cu) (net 18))
 (segment (start 74.458 100.6) (end 74.608 100.75) (width 1) (layer B.Cu) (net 17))
 (segment (start 72.15 100.6) (end 74.458 100.6) (width 1) (layer B.Cu) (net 17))
 (segment (start 74.608 100.75) (end 76 100.75) (width 1) (layer B.Cu) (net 17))
 (segment (start 76 100.75) (end 76 100.75) (width 1) (layer B.Cu) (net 17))
 (via (at 76 100.75) (size 1.2) (drill 0.7) (layers F.Cu B.Cu) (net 17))
 (segment (start 76 100.75) (end 77.25 102) (width 1) (layer F.Cu) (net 17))
 (segment (start 77.25 102) (end 77.25 102.75) (width 1) (layer F.Cu) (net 17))
 (segment (start 77.25 102.75) (end 77.25 103.25) (width 1) (layer F.Cu) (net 17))
 (segment (start 77.5 103.5) (end 77.25 103.25) (width 1) (layer F.Cu) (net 17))
 (segment (start 81.5 103.5) (end 77.5 103.5) (width 1) (layer F.Cu) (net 17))
 (segment (start 117.95 97.625) (end 118.075 97.75) (width 1) (layer F.Cu) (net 15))
 (segment (start 117.25 97.625) (end 117.95 97.625) (width 1) (layer F.Cu) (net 15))
 (segment (start 118.075 97.75) (end 119 97.75) (width 1) (layer F.Cu) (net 15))
 (segment (start 119 97.75) (end 119 97.75) (width 1) (layer F.Cu) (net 15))
 (via (at 119 97.75) (size 1.2) (drill 0.7) (layers F.Cu B.Cu) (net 15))
 (segment (start 130.5 97.75) (end 119 97.75) (width 1) (layer B.Cu) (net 15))
 (segment (start 141.25 87) (end 130.5 97.75) (width 1) (layer B.Cu) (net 15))
 (segment (start 150.676 73.778) (end 141.25 83.204) (width 1) (layer B.Cu) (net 15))
 (segment (start 141.25 83.204) (end 141.25 87) (width 1) (layer B.Cu) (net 15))
 (segment (start 105 79.42) (end 106.3 80.72) (width 0.5) (layer F.Cu) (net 5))
 (segment (start 105 73.5) (end 105 79.42) (width 0.5) (layer F.Cu) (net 5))
 (segment (start 112.113 80.72) (end 112.324 80.509) (width 1) (layer F.Cu) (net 5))
 (segment (start 106.3 80.72) (end 112.113 80.72) (width 1) (layer F.Cu) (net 5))
 (segment (start 134.79 67.29) (end 139.5 72) (width 1) (layer F.Cu) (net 10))
 (segment (start 134.79 66.5) (end 134.79 67.29) (width 1) (layer F.Cu) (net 10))
 (segment (start 129.7 66.49) (end 129.71 66.5) (width 1) (layer F.Cu) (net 4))
 (segment (start 129.71 63.365) (end 129.71 66.5) (width 1) (layer F.Cu) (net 4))
 (segment (start 130.7 63) (end 130.075 63) (width 1) (layer F.Cu) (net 4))
 (segment (start 130.075 63) (end 129.71 63.365) (width 1) (layer F.Cu) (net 4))
 (segment (start 127.5 71.25) (end 127.5 71.375) (width 0.5) (layer F.Cu) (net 11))
 (segment (start 132.25 66.5) (end 127.5 71.25) (width 0.5) (layer F.Cu) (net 11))
 (segment (start 124.757235 72) (end 125.5 71.257235) (width 1) (layer F.Cu) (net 11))
 (segment (start 123.5 72) (end 124.757235 72) (width 1) (layer F.Cu) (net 11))
 (segment (start 125.617765 71.375) (end 127.5 71.375) (width 1) (layer F.Cu) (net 11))
 (segment (start 125.5 71.257235) (end 125.617765 71.375) (width 1) (layer F.Cu) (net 11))
 (segment (start 139.5 82.287) (end 139.5 87) (width 1) (layer F.Cu) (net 8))
 (segment (start 139.5 87) (end 136.75 89.75) (width 1) (layer F.Cu) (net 8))
 (segment (start 129.46 89.25) (end 129.46 87.5) (width 1) (layer F.Cu) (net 8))
 (segment (start 129.96 89.75) (end 129.46 89.25) (width 1) (layer F.Cu) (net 8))
 (segment (start 136.75 89.75) (end 129.96 89.75) (width 1) (layer F.Cu) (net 8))
 (segment (start 133.5 83.5) (end 133.5 85) (width 1) (layer F.Cu) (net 3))
 (segment (start 134.54 86.04) (end 134.54 87.5) (width 1) (layer F.Cu) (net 3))
 (segment (start 133.5 85) (end 134.54 86.04) (width 1) (layer F.Cu) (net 3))
 (segment (start 127.463 82.287) (end 127.5 82.25) (width 0.5) (layer F.Cu) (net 9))
 (segment (start 123.5 82.287) (end 127.463 82.287) (width 0.5) (layer F.Cu) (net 9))
 (segment (start 127.5 83) (end 132 87.5) (width 0.5) (layer F.Cu) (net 9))
 (segment (start 127.5 82.25) (end 127.5 83) (width 0.5) (layer F.Cu) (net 9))
 (segment (start 95.25 103.5) (end 93.25 103.5) (width 1) (layer F.Cu) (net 13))
 (segment (start 91.625 101.875) (end 91.625 100.75) (width 1) (layer F.Cu) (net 13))
 (segment (start 93.25 103.5) (end 91.625 101.875) (width 1) (layer F.Cu) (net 13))
 (segment (start 91.625 97.5) (end 91.625 100.75) (width 1) (layer F.Cu) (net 13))
 (segment (start 90.005 95.88) (end 91.625 97.5) (width 1) (layer F.Cu) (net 13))
 (segment (start 89.12 95.88) (end 90.005 95.88) (width 1) (layer F.Cu) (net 13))
 (segment (start 142.96 89.075) (end 142.96 89.5625) (width 0.5) (layer F.Cu) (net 12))
 (segment (start 147.3935 89.5625) (end 148 88.956) (width 0.5) (layer F.Cu) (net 12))
 (segment (start 142.96 89.5625) (end 147.3935 89.5625) (width 0.5) (layer F.Cu) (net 12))
 (segment (start 151.144 92.1) (end 153.75 92.1) (width 0.5) (layer F.Cu) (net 12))
 (segment (start 148 88.956) (end 151.144 92.1) (width 0.5) (layer F.Cu) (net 12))
 (segment (start 139.5 75.683) (end 139.5 78.477) (width 1) (layer F.Cu) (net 12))
 (segment (start 148 87.698765) (end 148 88.956) (width 1) (layer F.Cu) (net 12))
 (segment (start 148 85.719765) (end 148 87.698765) (width 1) (layer F.Cu) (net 12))
 (segment (start 140.757235 78.477) (end 148 85.719765) (width 1) (layer F.Cu) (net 12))
 (segment (start 139.5 78.477) (end 140.757235 78.477) (width 1) (layer F.Cu) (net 12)))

